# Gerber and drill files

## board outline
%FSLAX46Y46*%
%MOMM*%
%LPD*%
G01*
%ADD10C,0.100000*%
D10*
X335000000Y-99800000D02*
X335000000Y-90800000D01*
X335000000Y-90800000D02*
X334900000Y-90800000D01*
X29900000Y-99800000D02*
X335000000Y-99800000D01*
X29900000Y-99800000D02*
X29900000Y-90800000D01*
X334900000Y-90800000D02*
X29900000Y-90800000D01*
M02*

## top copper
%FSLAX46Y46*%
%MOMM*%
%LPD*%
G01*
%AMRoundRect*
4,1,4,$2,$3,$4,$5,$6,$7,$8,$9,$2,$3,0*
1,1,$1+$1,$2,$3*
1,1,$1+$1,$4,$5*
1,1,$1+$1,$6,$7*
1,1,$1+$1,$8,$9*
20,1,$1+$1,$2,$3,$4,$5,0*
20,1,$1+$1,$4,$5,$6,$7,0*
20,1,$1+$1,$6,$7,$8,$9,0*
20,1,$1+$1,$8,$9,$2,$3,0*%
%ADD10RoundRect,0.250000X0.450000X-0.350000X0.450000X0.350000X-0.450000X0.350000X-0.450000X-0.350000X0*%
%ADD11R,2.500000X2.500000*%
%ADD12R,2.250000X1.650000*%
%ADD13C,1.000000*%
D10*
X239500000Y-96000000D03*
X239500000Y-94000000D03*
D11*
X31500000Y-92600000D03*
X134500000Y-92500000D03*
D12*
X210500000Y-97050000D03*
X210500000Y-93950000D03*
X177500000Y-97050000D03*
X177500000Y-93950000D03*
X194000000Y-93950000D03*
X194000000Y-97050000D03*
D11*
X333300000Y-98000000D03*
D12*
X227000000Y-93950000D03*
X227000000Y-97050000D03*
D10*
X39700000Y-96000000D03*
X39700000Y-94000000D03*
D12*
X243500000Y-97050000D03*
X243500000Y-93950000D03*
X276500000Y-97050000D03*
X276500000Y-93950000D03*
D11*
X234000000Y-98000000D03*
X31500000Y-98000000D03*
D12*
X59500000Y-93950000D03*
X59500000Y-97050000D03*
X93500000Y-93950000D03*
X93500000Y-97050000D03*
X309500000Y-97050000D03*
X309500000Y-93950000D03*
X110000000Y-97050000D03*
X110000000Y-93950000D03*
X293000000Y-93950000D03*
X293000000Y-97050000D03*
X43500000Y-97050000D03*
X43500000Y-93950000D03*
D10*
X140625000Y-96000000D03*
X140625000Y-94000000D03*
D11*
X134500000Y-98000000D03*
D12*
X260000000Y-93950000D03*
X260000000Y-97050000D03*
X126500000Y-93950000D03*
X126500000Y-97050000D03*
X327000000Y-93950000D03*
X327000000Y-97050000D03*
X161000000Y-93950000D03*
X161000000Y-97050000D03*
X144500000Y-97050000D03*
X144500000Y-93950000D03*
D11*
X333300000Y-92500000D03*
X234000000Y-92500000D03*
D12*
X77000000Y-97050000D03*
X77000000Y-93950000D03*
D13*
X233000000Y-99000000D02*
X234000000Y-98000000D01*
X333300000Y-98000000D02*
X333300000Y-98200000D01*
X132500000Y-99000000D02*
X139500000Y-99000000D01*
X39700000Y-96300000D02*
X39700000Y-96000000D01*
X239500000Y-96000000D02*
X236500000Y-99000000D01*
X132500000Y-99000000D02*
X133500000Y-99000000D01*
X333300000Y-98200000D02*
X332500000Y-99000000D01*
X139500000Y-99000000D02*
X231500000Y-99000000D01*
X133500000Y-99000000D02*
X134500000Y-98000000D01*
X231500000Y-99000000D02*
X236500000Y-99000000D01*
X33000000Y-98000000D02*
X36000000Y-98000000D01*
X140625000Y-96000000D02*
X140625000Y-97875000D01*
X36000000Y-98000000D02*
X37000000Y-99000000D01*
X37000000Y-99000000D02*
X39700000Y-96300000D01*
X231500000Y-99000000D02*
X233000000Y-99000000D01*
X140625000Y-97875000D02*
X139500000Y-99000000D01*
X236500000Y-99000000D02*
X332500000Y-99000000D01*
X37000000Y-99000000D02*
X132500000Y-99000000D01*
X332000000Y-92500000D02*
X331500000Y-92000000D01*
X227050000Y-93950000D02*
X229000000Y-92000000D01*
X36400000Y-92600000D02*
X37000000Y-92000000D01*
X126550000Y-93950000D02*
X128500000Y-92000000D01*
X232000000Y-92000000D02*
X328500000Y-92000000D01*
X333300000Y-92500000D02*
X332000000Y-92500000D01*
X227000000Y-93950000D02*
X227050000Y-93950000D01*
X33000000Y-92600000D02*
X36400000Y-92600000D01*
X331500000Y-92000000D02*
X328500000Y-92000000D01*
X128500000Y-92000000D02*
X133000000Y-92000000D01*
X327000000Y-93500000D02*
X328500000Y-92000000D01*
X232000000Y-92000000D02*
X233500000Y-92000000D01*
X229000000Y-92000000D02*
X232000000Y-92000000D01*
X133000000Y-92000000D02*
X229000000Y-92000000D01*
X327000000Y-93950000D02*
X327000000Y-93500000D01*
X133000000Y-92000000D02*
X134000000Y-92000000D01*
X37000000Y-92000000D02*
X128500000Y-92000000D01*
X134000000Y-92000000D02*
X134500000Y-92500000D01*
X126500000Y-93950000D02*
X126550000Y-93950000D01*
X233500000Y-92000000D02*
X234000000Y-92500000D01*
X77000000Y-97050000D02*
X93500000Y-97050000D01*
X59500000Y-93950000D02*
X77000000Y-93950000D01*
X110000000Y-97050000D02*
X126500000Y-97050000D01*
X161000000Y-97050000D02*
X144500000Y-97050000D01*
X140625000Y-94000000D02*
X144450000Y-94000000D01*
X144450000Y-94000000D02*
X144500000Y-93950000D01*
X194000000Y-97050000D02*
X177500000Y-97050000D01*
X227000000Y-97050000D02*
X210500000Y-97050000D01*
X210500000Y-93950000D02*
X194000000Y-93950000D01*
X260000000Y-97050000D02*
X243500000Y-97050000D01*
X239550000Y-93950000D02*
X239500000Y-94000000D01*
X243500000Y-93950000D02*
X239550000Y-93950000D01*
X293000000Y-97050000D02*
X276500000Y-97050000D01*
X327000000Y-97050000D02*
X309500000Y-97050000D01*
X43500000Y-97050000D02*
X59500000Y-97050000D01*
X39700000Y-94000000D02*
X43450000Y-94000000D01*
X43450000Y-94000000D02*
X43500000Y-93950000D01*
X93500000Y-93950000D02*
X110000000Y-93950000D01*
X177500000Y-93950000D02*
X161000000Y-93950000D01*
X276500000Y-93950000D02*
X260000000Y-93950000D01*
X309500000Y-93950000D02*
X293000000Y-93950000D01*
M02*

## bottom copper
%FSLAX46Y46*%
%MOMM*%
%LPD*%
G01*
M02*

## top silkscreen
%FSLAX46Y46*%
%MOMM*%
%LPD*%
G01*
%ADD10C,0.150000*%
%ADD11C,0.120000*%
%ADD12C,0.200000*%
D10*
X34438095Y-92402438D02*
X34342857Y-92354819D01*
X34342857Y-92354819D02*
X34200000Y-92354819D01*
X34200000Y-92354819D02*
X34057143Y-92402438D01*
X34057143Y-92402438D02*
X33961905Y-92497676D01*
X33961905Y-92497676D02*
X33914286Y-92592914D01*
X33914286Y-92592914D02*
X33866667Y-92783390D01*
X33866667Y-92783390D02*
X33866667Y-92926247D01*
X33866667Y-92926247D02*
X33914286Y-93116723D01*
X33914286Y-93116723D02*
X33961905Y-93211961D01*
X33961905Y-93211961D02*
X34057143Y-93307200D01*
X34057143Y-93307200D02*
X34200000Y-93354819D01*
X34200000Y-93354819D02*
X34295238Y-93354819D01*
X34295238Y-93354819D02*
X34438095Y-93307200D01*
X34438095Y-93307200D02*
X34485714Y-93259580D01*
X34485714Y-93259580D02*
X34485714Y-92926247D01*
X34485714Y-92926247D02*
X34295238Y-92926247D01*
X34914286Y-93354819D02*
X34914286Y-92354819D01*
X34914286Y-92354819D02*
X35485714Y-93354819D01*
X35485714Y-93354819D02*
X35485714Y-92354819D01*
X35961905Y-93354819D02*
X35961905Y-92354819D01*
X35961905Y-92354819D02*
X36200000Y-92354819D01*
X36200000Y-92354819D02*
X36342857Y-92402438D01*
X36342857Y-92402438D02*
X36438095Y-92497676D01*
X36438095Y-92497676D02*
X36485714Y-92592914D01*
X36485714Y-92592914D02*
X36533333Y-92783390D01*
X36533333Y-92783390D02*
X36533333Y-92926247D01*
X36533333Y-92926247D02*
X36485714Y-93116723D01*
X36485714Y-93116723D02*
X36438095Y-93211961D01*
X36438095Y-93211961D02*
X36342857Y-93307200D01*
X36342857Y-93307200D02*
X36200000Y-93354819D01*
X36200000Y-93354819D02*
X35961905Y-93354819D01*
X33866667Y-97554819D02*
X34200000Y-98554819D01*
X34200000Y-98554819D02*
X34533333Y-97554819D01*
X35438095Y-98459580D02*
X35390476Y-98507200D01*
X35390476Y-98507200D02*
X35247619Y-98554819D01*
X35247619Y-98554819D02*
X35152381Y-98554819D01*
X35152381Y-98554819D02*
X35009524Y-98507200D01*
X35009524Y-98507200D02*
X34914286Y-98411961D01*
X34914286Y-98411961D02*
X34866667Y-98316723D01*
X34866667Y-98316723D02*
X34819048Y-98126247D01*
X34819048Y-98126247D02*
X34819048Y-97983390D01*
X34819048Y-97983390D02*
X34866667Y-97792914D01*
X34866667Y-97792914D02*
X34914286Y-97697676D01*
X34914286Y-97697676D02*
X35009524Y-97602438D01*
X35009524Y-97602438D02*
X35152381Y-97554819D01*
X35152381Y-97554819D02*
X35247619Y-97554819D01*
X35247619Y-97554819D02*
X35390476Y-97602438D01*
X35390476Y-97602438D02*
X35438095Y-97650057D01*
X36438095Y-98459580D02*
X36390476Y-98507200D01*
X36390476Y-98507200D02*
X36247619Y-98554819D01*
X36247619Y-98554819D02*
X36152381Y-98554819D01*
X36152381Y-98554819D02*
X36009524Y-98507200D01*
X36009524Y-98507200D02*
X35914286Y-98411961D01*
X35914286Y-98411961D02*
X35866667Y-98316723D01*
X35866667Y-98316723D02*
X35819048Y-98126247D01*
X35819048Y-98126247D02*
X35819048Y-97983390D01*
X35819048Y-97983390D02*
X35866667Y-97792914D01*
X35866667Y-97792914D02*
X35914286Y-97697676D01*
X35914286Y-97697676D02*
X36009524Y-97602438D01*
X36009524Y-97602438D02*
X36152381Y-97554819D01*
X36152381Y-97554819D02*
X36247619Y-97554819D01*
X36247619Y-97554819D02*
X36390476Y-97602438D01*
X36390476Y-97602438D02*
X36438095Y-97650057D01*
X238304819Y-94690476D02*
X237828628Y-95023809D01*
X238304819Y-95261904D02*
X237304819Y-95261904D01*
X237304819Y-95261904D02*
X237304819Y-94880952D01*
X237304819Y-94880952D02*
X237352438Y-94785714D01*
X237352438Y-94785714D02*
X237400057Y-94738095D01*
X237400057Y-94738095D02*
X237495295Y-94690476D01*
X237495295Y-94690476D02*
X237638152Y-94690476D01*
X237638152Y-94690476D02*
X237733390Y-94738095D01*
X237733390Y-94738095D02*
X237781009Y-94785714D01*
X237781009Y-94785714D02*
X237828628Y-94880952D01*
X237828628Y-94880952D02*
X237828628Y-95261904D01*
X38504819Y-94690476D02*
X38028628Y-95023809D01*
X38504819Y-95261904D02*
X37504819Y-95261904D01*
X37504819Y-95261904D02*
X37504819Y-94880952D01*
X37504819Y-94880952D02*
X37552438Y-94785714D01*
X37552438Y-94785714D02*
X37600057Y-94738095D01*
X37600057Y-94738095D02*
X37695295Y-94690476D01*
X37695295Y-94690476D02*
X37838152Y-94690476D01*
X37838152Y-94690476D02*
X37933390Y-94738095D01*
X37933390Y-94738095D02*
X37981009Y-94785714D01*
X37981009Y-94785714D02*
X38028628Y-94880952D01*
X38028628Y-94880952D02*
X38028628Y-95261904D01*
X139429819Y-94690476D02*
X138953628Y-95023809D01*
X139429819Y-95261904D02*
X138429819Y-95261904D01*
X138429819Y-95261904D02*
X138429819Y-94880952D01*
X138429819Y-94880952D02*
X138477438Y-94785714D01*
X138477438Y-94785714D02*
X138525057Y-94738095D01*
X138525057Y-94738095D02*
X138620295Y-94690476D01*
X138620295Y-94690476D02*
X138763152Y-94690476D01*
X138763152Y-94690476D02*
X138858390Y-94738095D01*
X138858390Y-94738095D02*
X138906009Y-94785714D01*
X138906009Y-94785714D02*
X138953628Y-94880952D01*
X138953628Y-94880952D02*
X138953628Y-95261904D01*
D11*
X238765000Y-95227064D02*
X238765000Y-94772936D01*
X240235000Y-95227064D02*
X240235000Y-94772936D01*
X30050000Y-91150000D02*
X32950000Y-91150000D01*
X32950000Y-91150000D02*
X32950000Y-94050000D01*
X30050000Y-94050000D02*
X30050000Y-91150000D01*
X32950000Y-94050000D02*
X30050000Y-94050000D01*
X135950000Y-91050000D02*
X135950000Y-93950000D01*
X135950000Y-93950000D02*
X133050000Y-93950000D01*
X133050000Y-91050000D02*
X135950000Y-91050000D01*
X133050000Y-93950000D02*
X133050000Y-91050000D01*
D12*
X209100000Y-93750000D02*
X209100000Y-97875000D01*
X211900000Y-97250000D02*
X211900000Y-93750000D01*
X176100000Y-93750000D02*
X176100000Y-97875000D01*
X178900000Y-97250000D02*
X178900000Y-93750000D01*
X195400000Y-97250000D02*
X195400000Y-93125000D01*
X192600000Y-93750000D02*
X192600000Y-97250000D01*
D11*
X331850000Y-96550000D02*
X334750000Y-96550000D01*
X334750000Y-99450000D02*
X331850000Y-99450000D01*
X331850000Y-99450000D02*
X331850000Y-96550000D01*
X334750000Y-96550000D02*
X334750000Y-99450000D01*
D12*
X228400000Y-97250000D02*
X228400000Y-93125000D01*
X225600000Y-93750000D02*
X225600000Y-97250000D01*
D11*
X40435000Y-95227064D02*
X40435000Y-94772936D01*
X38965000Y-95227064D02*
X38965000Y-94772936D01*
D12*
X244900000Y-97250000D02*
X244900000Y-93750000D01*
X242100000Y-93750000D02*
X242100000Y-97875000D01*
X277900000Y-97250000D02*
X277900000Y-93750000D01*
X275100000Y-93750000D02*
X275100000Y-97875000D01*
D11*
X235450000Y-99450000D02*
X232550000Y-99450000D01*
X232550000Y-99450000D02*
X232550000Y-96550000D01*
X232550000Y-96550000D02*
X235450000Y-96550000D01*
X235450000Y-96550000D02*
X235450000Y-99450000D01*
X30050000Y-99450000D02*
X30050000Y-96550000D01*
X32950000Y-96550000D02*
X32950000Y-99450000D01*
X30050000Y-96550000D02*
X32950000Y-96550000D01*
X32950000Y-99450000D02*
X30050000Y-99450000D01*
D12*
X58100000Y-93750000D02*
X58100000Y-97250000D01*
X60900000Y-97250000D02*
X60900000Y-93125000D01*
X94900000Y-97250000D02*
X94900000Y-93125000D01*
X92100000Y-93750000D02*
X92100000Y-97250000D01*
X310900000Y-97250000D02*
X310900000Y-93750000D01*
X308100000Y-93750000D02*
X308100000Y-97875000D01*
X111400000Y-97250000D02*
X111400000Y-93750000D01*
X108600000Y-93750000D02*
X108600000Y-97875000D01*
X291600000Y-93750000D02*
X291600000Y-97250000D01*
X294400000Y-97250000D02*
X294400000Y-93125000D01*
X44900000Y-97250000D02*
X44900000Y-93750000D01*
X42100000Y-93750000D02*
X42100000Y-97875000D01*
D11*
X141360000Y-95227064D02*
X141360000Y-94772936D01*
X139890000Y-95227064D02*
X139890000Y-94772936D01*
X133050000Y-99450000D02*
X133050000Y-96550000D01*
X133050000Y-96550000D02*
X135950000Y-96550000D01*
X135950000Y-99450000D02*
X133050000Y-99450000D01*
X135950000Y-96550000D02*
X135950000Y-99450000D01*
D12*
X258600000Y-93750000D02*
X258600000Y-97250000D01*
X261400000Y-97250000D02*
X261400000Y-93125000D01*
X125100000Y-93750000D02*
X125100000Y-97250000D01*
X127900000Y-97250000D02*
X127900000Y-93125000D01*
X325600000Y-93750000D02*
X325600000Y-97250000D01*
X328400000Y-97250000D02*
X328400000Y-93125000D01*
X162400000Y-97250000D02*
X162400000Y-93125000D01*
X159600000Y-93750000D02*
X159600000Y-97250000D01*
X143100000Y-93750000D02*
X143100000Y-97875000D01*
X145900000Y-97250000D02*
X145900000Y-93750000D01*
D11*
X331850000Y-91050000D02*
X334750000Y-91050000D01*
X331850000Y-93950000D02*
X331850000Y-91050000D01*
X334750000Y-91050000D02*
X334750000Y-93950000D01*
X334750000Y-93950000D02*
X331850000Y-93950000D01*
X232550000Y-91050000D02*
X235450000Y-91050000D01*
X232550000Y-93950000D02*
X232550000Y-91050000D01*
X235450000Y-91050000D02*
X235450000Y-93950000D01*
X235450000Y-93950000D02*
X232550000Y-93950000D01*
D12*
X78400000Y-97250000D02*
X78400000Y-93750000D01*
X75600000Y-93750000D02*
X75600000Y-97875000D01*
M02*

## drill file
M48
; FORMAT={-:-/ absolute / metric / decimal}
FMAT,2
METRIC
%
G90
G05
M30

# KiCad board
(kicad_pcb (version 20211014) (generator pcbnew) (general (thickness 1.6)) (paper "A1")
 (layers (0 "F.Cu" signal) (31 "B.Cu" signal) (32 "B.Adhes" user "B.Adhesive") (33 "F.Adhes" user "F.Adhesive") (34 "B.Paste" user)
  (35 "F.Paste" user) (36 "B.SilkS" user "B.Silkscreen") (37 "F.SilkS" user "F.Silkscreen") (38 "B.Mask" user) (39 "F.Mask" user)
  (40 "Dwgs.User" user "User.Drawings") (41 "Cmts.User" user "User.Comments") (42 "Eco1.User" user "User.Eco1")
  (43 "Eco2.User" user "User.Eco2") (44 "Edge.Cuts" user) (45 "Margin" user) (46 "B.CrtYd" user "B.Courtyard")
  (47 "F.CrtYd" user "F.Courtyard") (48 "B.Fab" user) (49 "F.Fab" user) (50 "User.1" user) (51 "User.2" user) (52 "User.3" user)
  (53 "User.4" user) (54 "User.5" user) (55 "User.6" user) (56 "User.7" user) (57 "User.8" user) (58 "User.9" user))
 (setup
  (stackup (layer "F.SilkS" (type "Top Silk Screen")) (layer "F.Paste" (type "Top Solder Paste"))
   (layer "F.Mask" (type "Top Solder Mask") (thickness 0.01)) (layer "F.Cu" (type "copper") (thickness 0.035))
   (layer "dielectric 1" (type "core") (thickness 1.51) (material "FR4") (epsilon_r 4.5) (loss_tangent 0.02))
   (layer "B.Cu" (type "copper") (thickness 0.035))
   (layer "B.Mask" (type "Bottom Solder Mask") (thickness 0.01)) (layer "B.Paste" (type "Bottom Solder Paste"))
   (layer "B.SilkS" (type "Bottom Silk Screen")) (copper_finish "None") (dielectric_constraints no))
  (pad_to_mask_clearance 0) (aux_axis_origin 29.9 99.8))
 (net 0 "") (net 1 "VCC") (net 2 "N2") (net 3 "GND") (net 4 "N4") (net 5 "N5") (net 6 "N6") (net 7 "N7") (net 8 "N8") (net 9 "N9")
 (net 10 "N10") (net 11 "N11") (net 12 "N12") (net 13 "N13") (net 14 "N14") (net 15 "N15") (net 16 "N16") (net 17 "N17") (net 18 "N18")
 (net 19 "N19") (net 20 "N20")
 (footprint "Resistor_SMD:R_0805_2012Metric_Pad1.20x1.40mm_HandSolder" (layer "F.Cu") (at 239.5 95 90)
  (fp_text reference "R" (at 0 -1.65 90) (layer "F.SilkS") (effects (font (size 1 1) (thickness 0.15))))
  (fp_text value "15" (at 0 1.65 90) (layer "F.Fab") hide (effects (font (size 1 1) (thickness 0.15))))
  (fp_line (start -0.227064 -0.735) (end 0.227064 -0.735) (layer "F.SilkS") (width 0.12))
  (fp_line (start -0.227064 0.735) (end 0.227064 0.735) (layer "F.SilkS") (width 0.12))
  (pad "1" smd roundrect (at -1 0 90) (size 1.2 1.4) (layers "F.Cu" "F.Paste" "F.Mask") (roundrect_rratio 0.2083333333) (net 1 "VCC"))
  (pad "2" smd roundrect (at 1 0 90) (size 1.2 1.4) (layers "F.Cu" "F.Paste" "F.Mask") (roundrect_rratio 0.2083333333) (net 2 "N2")))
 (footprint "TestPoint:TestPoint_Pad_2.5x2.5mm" (layer "F.Cu") (at 31.5 92.6)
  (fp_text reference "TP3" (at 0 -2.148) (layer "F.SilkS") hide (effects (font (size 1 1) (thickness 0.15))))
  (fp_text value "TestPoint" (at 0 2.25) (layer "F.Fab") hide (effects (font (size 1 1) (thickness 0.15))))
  (fp_line (start -1.45 -1.45) (end 1.45 -1.45) (layer "F.SilkS") (width 0.12))
  (fp_line (start 1.45 -1.45) (end 1.45 1.45) (layer "F.SilkS") (width 0.12))
  (fp_line (start -1.45 1.45) (end -1.45 -1.45) (layer "F.SilkS") (width 0.12))
  (fp_line (start 1.45 1.45) (end -1.45 1.45) (layer "F.SilkS") (width 0.12))
  (pad "1" smd rect (at 0 0) (size 2.5 2.5) (layers "F.Cu" "F.Mask") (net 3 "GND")))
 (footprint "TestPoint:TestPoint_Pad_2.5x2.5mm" (layer "F.Cu") (at 134.5 92.5)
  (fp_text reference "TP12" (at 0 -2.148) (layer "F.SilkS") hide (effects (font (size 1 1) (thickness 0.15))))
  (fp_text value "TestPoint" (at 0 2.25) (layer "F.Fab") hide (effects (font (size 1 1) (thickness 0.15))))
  (fp_line (start 1.45 -1.45) (end 1.45 1.45) (layer "F.SilkS") (width 0.12))
  (fp_line (start 1.45 1.45) (end -1.45 1.45) (layer "F.SilkS") (width 0.12))
  (fp_line (start -1.45 -1.45) (end 1.45 -1.45) (layer "F.SilkS") (width 0.12))
  (fp_line (start -1.45 1.45) (end -1.45 -1.45) (layer "F.SilkS") (width 0.12))
  (pad "1" smd rect (at 0 0) (size 2.5 2.5) (layers "F.Cu" "F.Mask") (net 3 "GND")))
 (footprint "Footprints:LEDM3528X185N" (layer "F.Cu") (at 210.5 95.5 90)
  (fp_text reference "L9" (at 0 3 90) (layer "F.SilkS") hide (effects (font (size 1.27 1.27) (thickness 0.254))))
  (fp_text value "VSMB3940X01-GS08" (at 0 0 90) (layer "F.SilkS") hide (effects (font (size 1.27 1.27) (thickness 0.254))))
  (fp_line (start 1.75 -1.4) (end -2.375 -1.4) (layer "F.SilkS") (width 0.2))
  (fp_line (start -1.75 1.4) (end 1.75 1.4) (layer "F.SilkS") (width 0.2))
  (pad "1" smd rect (at -1.55 0 90) (size 1.65 2.25) (layers "F.Cu" "F.Paste" "F.Mask") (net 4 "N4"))
  (pad "2" smd rect (at 1.55 0 90) (size 1.65 2.25) (layers "F.Cu" "F.Paste" "F.Mask") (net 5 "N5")))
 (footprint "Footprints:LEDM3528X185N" (layer "F.Cu") (at 177.5 95.5 90)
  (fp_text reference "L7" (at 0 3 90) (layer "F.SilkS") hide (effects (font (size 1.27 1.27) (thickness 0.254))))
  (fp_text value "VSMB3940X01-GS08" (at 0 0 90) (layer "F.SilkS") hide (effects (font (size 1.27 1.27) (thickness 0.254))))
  (fp_line (start 1.75 -1.4) (end -2.375 -1.4) (layer "F.SilkS") (width 0.2))
  (fp_line (start -1.75 1.4) (end 1.75 1.4) (layer "F.SilkS") (width 0.2))
  (pad "1" smd rect (at -1.55 0 90) (size 1.65 2.25) (layers "F.Cu" "F.Paste" "F.Mask") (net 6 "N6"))
  (pad "2" smd rect (at 1.55 0 90) (size 1.65 2.25) (layers "F.Cu" "F.Paste" "F.Mask") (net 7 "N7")))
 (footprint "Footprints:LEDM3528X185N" (layer "F.Cu") (at 194 95.5 -90)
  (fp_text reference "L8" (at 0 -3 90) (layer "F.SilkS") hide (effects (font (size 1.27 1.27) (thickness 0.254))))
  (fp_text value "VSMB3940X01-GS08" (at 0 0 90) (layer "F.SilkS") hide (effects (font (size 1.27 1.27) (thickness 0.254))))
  (fp_line (start 1.75 -1.4) (end -2.375 -1.4) (layer "F.SilkS") (width 0.2))
  (fp_line (start -1.75 1.4) (end 1.75 1.4) (layer "F.SilkS") (width 0.2))
  (pad "1" smd rect (at -1.55 0 270) (size 1.65 2.25) (layers "F.Cu" "F.Paste" "F.Mask") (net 5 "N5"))
  (pad "2" smd rect (at 1.55 0 270) (size 1.65 2.25) (layers "F.Cu" "F.Paste" "F.Mask") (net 6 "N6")))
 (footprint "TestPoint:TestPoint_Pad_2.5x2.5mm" (layer "F.Cu") (at 333.3 98)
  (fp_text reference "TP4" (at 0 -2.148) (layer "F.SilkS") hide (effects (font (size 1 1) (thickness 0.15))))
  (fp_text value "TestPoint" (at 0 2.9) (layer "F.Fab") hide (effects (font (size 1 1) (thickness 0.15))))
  (fp_line (start -1.45 -1.45) (end 1.45 -1.45) (layer "F.SilkS") (width 0.12))
  (fp_line (start 1.45 1.45) (end -1.45 1.45) (layer "F.SilkS") (width 0.12))
  (fp_line (start -1.45 1.45) (end -1.45 -1.45) (layer "F.SilkS") (width 0.12))
  (fp_line (start 1.45 -1.45) (end 1.45 1.45) (layer "F.SilkS") (width 0.12))
  (pad "1" smd rect (at 0 0) (size 2.5 2.5) (layers "F.Cu" "F.Mask") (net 1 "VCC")))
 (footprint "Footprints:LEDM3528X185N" (layer "F.Cu") (at 227 95.5 -90)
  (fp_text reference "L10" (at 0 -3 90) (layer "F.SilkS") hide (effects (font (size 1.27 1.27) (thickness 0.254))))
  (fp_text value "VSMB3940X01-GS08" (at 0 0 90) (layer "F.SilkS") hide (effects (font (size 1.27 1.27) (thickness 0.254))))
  (fp_line (start 1.75 -1.4) (end -2.375 -1.4) (layer "F.SilkS") (width 0.2))
  (fp_line (start -1.75 1.4) (end 1.75 1.4) (layer "F.SilkS") (width 0.2))
  (pad "1" smd rect (at -1.55 0 270) (size 1.65 2.25) (layers "F.Cu" "F.Paste" "F.Mask") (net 3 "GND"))
  (pad "2" smd rect (at 1.55 0 270) (size 1.65 2.25) (layers "F.Cu" "F.Paste" "F.Mask") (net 4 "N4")))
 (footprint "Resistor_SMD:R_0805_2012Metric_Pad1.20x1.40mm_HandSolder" (layer "F.Cu") (at 39.7 95 90)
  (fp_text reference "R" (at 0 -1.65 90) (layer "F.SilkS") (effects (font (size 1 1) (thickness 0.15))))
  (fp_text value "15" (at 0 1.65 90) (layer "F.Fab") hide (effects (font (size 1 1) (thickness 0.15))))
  (fp_line (start -0.227064 0.735) (end 0.227064 0.735) (layer "F.SilkS") (width 0.12))
  (fp_line (start -0.227064 -0.735) (end 0.227064 -0.735) (layer "F.SilkS") (width 0.12))
  (pad "1" smd roundrect (at -1 0 90) (size 1.2 1.4) (layers "F.Cu" "F.Paste" "F.Mask") (roundrect_rratio 0.2083333333) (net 1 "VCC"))
  (pad "2" smd roundrect (at 1 0 90) (size 1.2 1.4) (layers "F.Cu" "F.Paste" "F.Mask") (roundrect_rratio 0.2083333333) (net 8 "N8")))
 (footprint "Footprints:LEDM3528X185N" (layer "F.Cu") (at 243.5 95.5 90)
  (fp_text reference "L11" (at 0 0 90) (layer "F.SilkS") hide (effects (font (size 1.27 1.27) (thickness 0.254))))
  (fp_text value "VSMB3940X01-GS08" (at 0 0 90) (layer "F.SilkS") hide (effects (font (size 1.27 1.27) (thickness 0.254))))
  (fp_line (start -1.75 1.4) (end 1.75 1.4) (layer "F.SilkS") (width 0.2))
  (fp_line (start 1.75 -1.4) (end -2.375 -1.4) (layer "F.SilkS") (width 0.2))
  (pad "1" smd rect (at -1.55 0 90) (size 1.65 2.25) (layers "F.Cu" "F.Paste" "F.Mask") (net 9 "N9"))
  (pad "2" smd rect (at 1.55 0 90) (size 1.65 2.25) (layers "F.Cu" "F.Paste" "F.Mask") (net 2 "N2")))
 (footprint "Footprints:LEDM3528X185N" (layer "F.Cu") (at 276.5 95.5 90)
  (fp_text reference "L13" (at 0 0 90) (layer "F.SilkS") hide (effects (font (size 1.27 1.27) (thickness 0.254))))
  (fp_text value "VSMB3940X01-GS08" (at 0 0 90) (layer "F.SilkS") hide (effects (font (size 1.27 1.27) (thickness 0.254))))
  (fp_line (start -1.75 1.4) (end 1.75 1.4) (layer "F.SilkS") (width 0.2))
  (fp_line (start 1.75 -1.4) (end -2.375 -1.4) (layer "F.SilkS") (width 0.2))
  (pad "1" smd rect (at -1.55 0 90) (size 1.65 2.25) (layers "F.Cu" "F.Paste" "F.Mask") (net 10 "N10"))
  (pad "2" smd rect (at 1.55 0 90) (size 1.65 2.25) (layers "F.Cu" "F.Paste" "F.Mask") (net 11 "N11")))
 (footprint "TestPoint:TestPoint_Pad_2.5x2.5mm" (layer "F.Cu") (at 234 98)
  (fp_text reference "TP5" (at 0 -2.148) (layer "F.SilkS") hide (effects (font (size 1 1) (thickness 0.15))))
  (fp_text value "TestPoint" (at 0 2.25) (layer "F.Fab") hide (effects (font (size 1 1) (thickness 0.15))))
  (fp_line (start 1.45 1.45) (end -1.45 1.45) (layer "F.SilkS") (width 0.12))
  (fp_line (start -1.45 1.45) (end -1.45 -1.45) (layer "F.SilkS") (width 0.12))
  (fp_line (start -1.45 -1.45) (end 1.45 -1.45) (layer "F.SilkS") (width 0.12))
  (fp_line (start 1.45 -1.45) (end 1.45 1.45) (layer "F.SilkS") (width 0.12))
  (pad "1" smd rect (at 0 0) (size 2.5 2.5) (layers "F.Cu" "F.Mask") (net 1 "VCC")))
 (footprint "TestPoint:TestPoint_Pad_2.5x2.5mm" (layer "F.Cu") (at 31.5 98)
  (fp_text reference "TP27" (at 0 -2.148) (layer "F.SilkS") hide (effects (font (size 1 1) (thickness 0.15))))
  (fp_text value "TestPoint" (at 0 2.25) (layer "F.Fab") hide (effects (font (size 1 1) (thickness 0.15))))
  (fp_line (start -1.45 1.45) (end -1.45 -1.45) (layer "F.SilkS") (width 0.12))
  (fp_line (start 1.45 -1.45) (end 1.45 1.45) (layer "F.SilkS") (width 0.12))
  (fp_line (start -1.45 -1.45) (end 1.45 -1.45) (layer "F.SilkS") (width 0.12))
  (fp_line (start 1.45 1.45) (end -1.45 1.45) (layer "F.SilkS") (width 0.12))
  (pad "1" smd rect (at 0 0) (size 2.5 2.5) (layers "F.Cu" "F.Mask") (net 1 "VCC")))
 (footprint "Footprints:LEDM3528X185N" (layer "F.Cu") (at 59.5 95.5 -90)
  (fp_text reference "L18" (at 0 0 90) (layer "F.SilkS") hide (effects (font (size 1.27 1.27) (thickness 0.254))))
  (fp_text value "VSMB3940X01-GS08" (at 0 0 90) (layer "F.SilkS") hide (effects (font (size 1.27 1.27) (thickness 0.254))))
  (fp_line (start -1.75 1.4) (end 1.75 1.4) (layer "F.SilkS") (width 0.2))
  (fp_line (start 1.75 -1.4) (end -2.375 -1.4) (layer "F.SilkS") (width 0.2))
  (pad "1" smd rect (at -1.55 0 270) (size 1.65 2.25) (layers "F.Cu" "F.Paste" "F.Mask") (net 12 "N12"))
  (pad "2" smd rect (at 1.55 0 270) (size 1.65 2.25) (layers "F.Cu" "F.Paste" "F.Mask") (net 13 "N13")))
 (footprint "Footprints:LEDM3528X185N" (layer "F.Cu") (at 93.5 95.5 -90)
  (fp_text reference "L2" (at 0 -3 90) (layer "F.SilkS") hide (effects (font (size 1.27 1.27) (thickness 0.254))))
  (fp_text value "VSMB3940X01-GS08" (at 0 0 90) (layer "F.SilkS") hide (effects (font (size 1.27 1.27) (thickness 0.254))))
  (fp_line (start 1.75 -1.4) (end -2.375 -1.4) (layer "F.SilkS") (width 0.2))
  (fp_line (start -1.75 1.4) (end 1.75 1.4) (layer "F.SilkS") (width 0.2))
  (pad "1" smd rect (at -1.55 0 270) (size 1.65 2.25) (layers "F.Cu" "F.Paste" "F.Mask") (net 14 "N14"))
  (pad "2" smd rect (at 1.55 0 270) (size 1.65 2.25) (layers "F.Cu" "F.Paste" "F.Mask") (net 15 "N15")))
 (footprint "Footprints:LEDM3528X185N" (layer "F.Cu") (at 309.5 95.5 90)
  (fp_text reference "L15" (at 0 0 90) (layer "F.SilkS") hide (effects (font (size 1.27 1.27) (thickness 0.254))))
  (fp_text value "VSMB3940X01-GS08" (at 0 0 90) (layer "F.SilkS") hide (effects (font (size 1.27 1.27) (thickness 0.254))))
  (fp_line (start -1.75 1.4) (end 1.75 1.4) (layer "F.SilkS") (width 0.2))
  (fp_line (start 1.75 -1.4) (end -2.375 -1.4) (layer "F.SilkS") (width 0.2))
  (pad "1" smd rect (at -1.55 0 90) (size 1.65 2.25) (layers "F.Cu" "F.Paste" "F.Mask") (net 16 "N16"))
  (pad "2" smd rect (at 1.55 0 90) (size 1.65 2.25) (layers "F.Cu" "F.Paste" "F.Mask") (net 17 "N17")))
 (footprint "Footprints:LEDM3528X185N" (layer "F.Cu") (at 110 95.5 90)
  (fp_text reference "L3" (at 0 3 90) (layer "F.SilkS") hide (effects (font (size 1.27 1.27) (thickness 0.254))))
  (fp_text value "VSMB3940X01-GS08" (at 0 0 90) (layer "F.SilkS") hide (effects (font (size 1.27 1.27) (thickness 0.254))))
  (fp_line (start -1.75 1.4) (end 1.75 1.4) (layer "F.SilkS") (width 0.2))
  (fp_line (start 1.75 -1.4) (end -2.375 -1.4) (layer "F.SilkS") (width 0.2))
  (pad "1" smd rect (at -1.55 0 90) (size 1.65 2.25) (layers "F.Cu" "F.Paste" "F.Mask") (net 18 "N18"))
  (pad "2" smd rect (at 1.55 0 90) (size 1.65 2.25) (layers "F.Cu" "F.Paste" "F.Mask") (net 14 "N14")))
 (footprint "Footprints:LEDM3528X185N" (layer "F.Cu") (at 293 95.5 -90)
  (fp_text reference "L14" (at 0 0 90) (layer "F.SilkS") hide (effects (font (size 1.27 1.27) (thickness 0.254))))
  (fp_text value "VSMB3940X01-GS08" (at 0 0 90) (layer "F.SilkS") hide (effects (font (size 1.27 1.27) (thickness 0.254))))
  (fp_line (start -1.75 1.4) (end 1.75 1.4) (layer "F.SilkS") (width 0.2))
  (fp_line (start 1.75 -1.4) (end -2.375 -1.4) (layer "F.SilkS") (width 0.2))
  (pad "1" smd rect (at -1.55 0 270) (size 1.65 2.25) (layers "F.Cu" "F.Paste" "F.Mask") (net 17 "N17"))
  (pad "2" smd rect (at 1.55 0 270) (size 1.65 2.25) (layers "F.Cu" "F.Paste" "F.Mask") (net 10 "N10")))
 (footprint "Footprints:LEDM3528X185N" (layer "F.Cu") (at 43.5 95.5 90)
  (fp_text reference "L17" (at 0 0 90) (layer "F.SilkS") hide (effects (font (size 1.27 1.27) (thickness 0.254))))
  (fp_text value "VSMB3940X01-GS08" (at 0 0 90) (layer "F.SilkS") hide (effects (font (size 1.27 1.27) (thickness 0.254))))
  (fp_line (start -1.75 1.4) (end 1.75 1.4) (layer "F.SilkS") (width 0.2))
  (fp_line (start 1.75 -1.4) (end -2.375 -1.4) (layer "F.SilkS") (width 0.2))
  (pad "1" smd rect (at -1.55 0 90) (size 1.65 2.25) (layers "F.Cu" "F.Paste" "F.Mask") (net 13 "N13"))
  (pad "2" smd rect (at 1.55 0 90) (size 1.65 2.25) (layers "F.Cu" "F.Paste" "F.Mask") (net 8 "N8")))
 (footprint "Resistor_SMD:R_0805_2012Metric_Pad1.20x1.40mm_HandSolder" (layer "F.Cu") (at 140.625 95 90)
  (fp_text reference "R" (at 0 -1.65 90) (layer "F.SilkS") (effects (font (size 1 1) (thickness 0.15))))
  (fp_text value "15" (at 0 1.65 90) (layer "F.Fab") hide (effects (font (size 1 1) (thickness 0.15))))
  (fp_line (start -0.227064 0.735) (end 0.227064 0.735) (layer "F.SilkS") (width 0.12))
  (fp_line (start -0.227064 -0.735) (end 0.227064 -0.735) (layer "F.SilkS") (width 0.12))
  (pad "1" smd roundrect (at -1 0 90) (size 1.2 1.4) (layers "F.Cu" "F.Paste" "F.Mask") (roundrect_rratio 0.2083333333) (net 1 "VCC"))
  (pad "2" smd roundrect (at 1 0 90) (size 1.2 1.4) (layers "F.Cu" "F.Paste" "F.Mask") (roundrect_rratio 0.2083333333) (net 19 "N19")))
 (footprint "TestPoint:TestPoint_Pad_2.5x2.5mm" (layer "F.Cu") (at 134.5 98)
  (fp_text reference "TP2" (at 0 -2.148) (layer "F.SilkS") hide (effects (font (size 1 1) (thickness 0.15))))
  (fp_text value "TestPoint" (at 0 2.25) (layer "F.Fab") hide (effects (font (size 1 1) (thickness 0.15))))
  (fp_line (start -1.45 1.45) (end -1.45 -1.45) (layer "F.SilkS") (width 0.12))
  (fp_line (start -1.45 -1.45) (end 1.45 -1.45) (layer "F.SilkS") (width 0.12))
  (fp_line (start 1.45 1.45) (end -1.45 1.45) (layer "F.SilkS") (width 0.12))
  (fp_line (start 1.45 -1.45) (end 1.45 1.45) (layer "F.SilkS") (width 0.12))
  (pad "1" smd rect (at 0 0) (size 2.5 2.5) (layers "F.Cu" "F.Mask") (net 1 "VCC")))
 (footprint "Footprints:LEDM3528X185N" (layer "F.Cu") (at 260 95.5 -90)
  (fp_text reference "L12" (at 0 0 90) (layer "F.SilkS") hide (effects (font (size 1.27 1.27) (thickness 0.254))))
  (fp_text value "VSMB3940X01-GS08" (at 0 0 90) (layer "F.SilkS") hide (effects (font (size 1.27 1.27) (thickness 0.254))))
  (fp_line (start -1.75 1.4) (end 1.75 1.4) (layer "F.SilkS") (width 0.2))
  (fp_line (start 1.75 -1.4) (end -2.375 -1.4) (layer "F.SilkS") (width 0.2))
  (pad "1" smd rect (at -1.55 0 270) (size 1.65 2.25) (layers "F.Cu" "F.Paste" "F.Mask") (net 11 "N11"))
  (pad "2" smd rect (at 1.55 0 270) (size 1.65 2.25) (layers "F.Cu" "F.Paste" "F.Mask") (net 9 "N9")))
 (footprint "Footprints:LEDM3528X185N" (layer "F.Cu") (at 126.5 95.5 -90)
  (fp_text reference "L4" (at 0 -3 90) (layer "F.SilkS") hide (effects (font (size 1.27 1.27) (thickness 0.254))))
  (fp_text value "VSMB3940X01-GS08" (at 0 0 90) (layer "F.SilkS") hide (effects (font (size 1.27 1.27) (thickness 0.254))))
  (fp_line (start -1.75 1.4) (end 1.75 1.4) (layer "F.SilkS") (width 0.2))
  (fp_line (start 1.75 -1.4) (end -2.375 -1.4) (layer "F.SilkS") (width 0.2))
  (pad "1" smd rect (at -1.55 0 270) (size 1.65 2.25) (layers "F.Cu" "F.Paste" "F.Mask") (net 3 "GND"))
  (pad "2" smd rect (at 1.55 0 270) (size 1.65 2.25) (layers "F.Cu" "F.Paste" "F.Mask") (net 18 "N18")))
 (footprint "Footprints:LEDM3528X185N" (layer "F.Cu") (at 327 95.5 -90)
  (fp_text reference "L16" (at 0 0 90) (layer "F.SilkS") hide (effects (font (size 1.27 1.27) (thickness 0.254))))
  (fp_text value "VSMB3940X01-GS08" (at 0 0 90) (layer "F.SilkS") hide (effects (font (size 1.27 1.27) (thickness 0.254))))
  (fp_line (start -1.75 1.4) (end 1.75 1.4) (layer "F.SilkS") (width 0.2))
  (fp_line (start 1.75 -1.4) (end -2.375 -1.4) (layer "F.SilkS") (width 0.2))
  (pad "1" smd rect (at -1.55 0 270) (size 1.65 2.25) (layers "F.Cu" "F.Paste" "F.Mask") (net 3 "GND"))
  (pad "2" smd rect (at 1.55 0 270) (size 1.65 2.25) (layers "F.Cu" "F.Paste" "F.Mask") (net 16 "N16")))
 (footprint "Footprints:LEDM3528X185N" (layer "F.Cu") (at 161 95.5 -90)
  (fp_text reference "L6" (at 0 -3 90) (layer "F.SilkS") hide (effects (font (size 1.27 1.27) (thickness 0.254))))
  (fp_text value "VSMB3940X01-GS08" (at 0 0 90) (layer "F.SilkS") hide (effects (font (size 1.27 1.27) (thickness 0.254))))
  (fp_line (start 1.75 -1.4) (end -2.375 -1.4) (layer "F.SilkS") (width 0.2))
  (fp_line (start -1.75 1.4) (end 1.75 1.4) (layer "F.SilkS") (width 0.2))
  (pad "1" smd rect (at -1.55 0 270) (size 1.65 2.25) (layers "F.Cu" "F.Paste" "F.Mask") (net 7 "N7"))
  (pad "2" smd rect (at 1.55 0 270) (size 1.65 2.25) (layers "F.Cu" "F.Paste" "F.Mask") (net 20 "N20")))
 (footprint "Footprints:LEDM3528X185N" (layer "F.Cu") (at 144.5 95.5 90)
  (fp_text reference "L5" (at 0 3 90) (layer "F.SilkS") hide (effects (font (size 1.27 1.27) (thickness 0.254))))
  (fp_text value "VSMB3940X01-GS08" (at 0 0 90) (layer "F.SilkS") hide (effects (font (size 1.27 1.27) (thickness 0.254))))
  (fp_line (start 1.75 -1.4) (end -2.375 -1.4) (layer "F.SilkS") (width 0.2))
  (fp_line (start -1.75 1.4) (end 1.75 1.4) (layer "F.SilkS") (width 0.2))
  (pad "1" smd rect (at -1.55 0 90) (size 1.65 2.25) (layers "F.Cu" "F.Paste" "F.Mask") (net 20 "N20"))
  (pad "2" smd rect (at 1.55 0 90) (size 1.65 2.25) (layers "F.Cu" "F.Paste" "F.Mask") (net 19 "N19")))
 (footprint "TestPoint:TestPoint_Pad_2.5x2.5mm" (layer "F.Cu") (at 333.3 92.5)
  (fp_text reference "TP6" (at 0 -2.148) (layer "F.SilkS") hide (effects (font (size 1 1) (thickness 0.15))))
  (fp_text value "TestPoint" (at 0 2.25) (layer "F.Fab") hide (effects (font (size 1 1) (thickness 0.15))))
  (fp_line (start -1.45 -1.45) (end 1.45 -1.45) (layer "F.SilkS") (width 0.12))
  (fp_line (start -1.45 1.45) (end -1.45 -1.45) (layer "F.SilkS") (width 0.12))
  (fp_line (start 1.45 -1.45) (end 1.45 1.45) (layer "F.SilkS") (width 0.12))
  (fp_line (start 1.45 1.45) (end -1.45 1.45) (layer "F.SilkS") (width 0.12))
  (pad "1" smd rect (at 0 0) (size 2.5 2.5) (layers "F.Cu" "F.Mask") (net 3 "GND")))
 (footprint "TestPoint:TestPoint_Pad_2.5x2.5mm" (layer "F.Cu") (at 234 92.5)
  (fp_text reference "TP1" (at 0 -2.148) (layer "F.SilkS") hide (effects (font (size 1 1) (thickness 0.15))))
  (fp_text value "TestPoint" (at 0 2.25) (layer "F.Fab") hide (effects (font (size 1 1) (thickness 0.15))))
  (fp_line (start -1.45 -1.45) (end 1.45 -1.45) (layer "F.SilkS") (width 0.12))
  (fp_line (start -1.45 1.45) (end -1.45 -1.45) (layer "F.SilkS") (width 0.12))
  (fp_line (start 1.45 -1.45) (end 1.45 1.45) (layer "F.SilkS") (width 0.12))
  (fp_line (start 1.45 1.45) (end -1.45 1.45) (layer "F.SilkS") (width 0.12))
  (pad "1" smd rect (at 0 0) (size 2.5 2.5) (layers "F.Cu" "F.Mask") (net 3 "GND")))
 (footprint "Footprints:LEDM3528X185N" (layer "F.Cu") (at 77 95.5 90)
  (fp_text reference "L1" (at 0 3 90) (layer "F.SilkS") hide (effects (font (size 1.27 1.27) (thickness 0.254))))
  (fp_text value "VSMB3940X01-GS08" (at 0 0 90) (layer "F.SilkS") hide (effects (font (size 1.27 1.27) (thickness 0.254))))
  (fp_line (start -1.75 1.4) (end 1.75 1.4) (layer "F.SilkS") (width 0.2))
  (fp_line (start 1.75 -1.4) (end -2.375 -1.4) (layer "F.SilkS") (width 0.2))
  (pad "1" smd rect (at -1.55 0 90) (size 1.65 2.25) (layers "F.Cu" "F.Paste" "F.Mask") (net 15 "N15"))
  (pad "2" smd rect (at 1.55 0 90) (size 1.65 2.25) (layers "F.Cu" "F.Paste" "F.Mask") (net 12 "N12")))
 (gr_line (start 335 99.8) (end 335 90.8) (layer "Edge.Cuts") (width 0.1))
 (gr_line (start 335 90.8) (end 334.9 90.8) (layer "Edge.Cuts") (width 0.1))
 (gr_line (start 29.9 99.8) (end 335 99.8) (layer "Edge.Cuts") (width 0.1))
 (gr_line (start 29.9 99.8) (end 29.9 90.8) (layer "Edge.Cuts") (width 0.1))
 (gr_line (start 334.9 90.8) (end 29.9 90.8) (layer "Edge.Cuts") (width 0.1))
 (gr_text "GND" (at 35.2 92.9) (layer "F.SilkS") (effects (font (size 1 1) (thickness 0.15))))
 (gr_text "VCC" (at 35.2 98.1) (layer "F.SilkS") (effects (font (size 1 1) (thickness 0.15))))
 (segment (start 233 99) (end 234 98) (width 1) (layer "F.Cu") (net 1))
 (segment (start 333.3 98) (end 333.3 98.2) (width 1) (layer "F.Cu") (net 1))
 (segment (start 132.5 99) (end 139.5 99) (width 1) (layer "F.Cu") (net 1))
 (segment (start 39.7 96.3) (end 39.7 96) (width 1) (layer "F.Cu") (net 1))
 (segment (start 239.5 96) (end 236.5 99) (width 1) (layer "F.Cu") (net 1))
 (segment (start 132.5 99) (end 133.5 99) (width 1) (layer "F.Cu") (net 1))
 (segment (start 333.3 98.2) (end 332.5 99) (width 1) (layer "F.Cu") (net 1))
 (segment (start 139.5 99) (end 231.5 99) (width 1) (layer "F.Cu") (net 1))
 (segment (start 133.5 99) (end 134.5 98) (width 1) (layer "F.Cu") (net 1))
 (segment (start 231.5 99) (end 236.5 99) (width 1) (layer "F.Cu") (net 1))
 (segment (start 33 98) (end 36 98) (width 1) (layer "F.Cu") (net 1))
 (segment (start 140.625 96) (end 140.625 97.875) (width 1) (layer "F.Cu") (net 1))
 (segment (start 36 98) (end 37 99) (width 1) (layer "F.Cu") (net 1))
 (segment (start 37 99) (end 39.7 96.3) (width 1) (layer "F.Cu") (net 1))
 (segment (start 231.5 99) (end 233 99) (width 1) (layer "F.Cu") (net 1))
 (segment (start 140.625 97.875) (end 139.5 99) (width 1) (layer "F.Cu") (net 1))
 (segment (start 236.5 99) (end 332.5 99) (width 1) (layer "F.Cu") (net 1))
 (segment (start 37 99) (end 132.5 99) (width 1) (layer "F.Cu") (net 1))
 (segment (start 332 92.5) (end 331.5 92) (width 1) (layer "F.Cu") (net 3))
 (segment (start 227.05 93.95) (end 229 92) (width 1) (layer "F.Cu") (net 3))
 (segment (start 36.4 92.6) (end 37 92) (width 1) (layer "F.Cu") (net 3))
 (segment (start 126.55 93.95) (end 128.5 92) (width 1) (layer "F.Cu") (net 3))
 (segment (start 232 92) (end 328.5 92) (width 1) (layer "F.Cu") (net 3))
 (segment (start 333.3 92.5) (end 332 92.5) (width 1) (layer "F.Cu") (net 3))
 (segment (start 227 93.95) (end 227.05 93.95) (width 1) (layer "F.Cu") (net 3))
 (segment (start 33 92.6) (end 36.4 92.6) (width 1) (layer "F.Cu") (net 3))
 (segment (start 331.5 92) (end 328.5 92) (width 1) (layer "F.Cu") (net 3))
 (segment (start 128.5 92) (end 133 92) (width 1) (layer "F.Cu") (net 3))
 (segment (start 327 93.5) (end 328.5 92) (width 1) (layer "F.Cu") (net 3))
 (segment (start 232 92) (end 233.5 92) (width 1) (layer "F.Cu") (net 3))
 (segment (start 229 92) (end 232 92) (width 1) (layer "F.Cu") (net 3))
 (segment (start 133 92) (end 229 92) (width 1) (layer "F.Cu") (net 3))
 (segment (start 327 93.95) (end 327 93.5) (width 1) (layer "F.Cu") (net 3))
 (segment (start 133 92) (end 134 92) (width 1) (layer "F.Cu") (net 3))
 (segment (start 37 92) (end 128.5 92) (width 1) (layer "F.Cu") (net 3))
 (segment (start 134 92) (end 134.5 92.5) (width 1) (layer "F.Cu") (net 3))
 (segment (start 126.5 93.95) (end 126.55 93.95) (width 1) (layer "F.Cu") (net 3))
 (segment (start 233.5 92) (end 234 92.5) (width 1) (layer "F.Cu") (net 3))
 (segment (start 77 97.05) (end 93.5 97.05) (width 1) (layer "F.Cu") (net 15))
 (segment (start 59.5 93.95) (end 77 93.95) (width 1) (layer "F.Cu") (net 12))
 (segment (start 110 97.05) (end 126.5 97.05) (width 1) (layer "F.Cu") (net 18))
 (segment (start 161 97.05) (end 144.5 97.05) (width 1) (layer "F.Cu") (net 20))
 (segment (start 140.625 94) (end 144.45 94) (width 1) (layer "F.Cu") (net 19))
 (segment (start 144.45 94) (end 144.5 93.95) (width 1) (layer "F.Cu") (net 19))
 (segment (start 194 97.05) (end 177.5 97.05) (width 1) (layer "F.Cu") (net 6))
 (segment (start 227 97.05) (end 210.5 97.05) (width 1) (layer "F.Cu") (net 4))
 (segment (start 210.5 93.95) (end 194 93.95) (width 1) (layer "F.Cu") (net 5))
 (segment (start 260 97.05) (end 243.5 97.05) (width 1) (layer "F.Cu") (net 9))
 (segment (start 239.55 93.95) (end 239.5 94) (width 1) (layer "F.Cu") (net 2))
 (segment (start 243.5 93.95) (end 239.55 93.95) (width 1) (layer "F.Cu") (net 2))
 (segment (start 293 97.05) (end 276.5 97.05) (width 1) (layer "F.Cu") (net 10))
 (segment (start 327 97.05) (end 309.5 97.05) (width 1) (layer "F.Cu") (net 16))
 (segment (start 43.5 97.05) (end 59.5 97.05) (width 1) (layer "F.Cu") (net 13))
 (segment (start 39.7 94) (end 43.45 94) (width 1) (layer "F.Cu") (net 8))
 (segment (start 43.45 94) (end 43.5 93.95) (width 1) (layer "F.Cu") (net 8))
 (segment (start 93.5 93.95) (end 110 93.95) (width 1) (layer "F.Cu") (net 14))
 (segment (start 177.5 93.95) (end 161 93.95) (width 1) (layer "F.Cu") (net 7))
 (segment (start 276.5 93.95) (end 260 93.95) (width 1) (layer "F.Cu") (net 11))
 (segment (start 309.5 93.95) (end 293 93.95) (width 1) (layer "F.Cu") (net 17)))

